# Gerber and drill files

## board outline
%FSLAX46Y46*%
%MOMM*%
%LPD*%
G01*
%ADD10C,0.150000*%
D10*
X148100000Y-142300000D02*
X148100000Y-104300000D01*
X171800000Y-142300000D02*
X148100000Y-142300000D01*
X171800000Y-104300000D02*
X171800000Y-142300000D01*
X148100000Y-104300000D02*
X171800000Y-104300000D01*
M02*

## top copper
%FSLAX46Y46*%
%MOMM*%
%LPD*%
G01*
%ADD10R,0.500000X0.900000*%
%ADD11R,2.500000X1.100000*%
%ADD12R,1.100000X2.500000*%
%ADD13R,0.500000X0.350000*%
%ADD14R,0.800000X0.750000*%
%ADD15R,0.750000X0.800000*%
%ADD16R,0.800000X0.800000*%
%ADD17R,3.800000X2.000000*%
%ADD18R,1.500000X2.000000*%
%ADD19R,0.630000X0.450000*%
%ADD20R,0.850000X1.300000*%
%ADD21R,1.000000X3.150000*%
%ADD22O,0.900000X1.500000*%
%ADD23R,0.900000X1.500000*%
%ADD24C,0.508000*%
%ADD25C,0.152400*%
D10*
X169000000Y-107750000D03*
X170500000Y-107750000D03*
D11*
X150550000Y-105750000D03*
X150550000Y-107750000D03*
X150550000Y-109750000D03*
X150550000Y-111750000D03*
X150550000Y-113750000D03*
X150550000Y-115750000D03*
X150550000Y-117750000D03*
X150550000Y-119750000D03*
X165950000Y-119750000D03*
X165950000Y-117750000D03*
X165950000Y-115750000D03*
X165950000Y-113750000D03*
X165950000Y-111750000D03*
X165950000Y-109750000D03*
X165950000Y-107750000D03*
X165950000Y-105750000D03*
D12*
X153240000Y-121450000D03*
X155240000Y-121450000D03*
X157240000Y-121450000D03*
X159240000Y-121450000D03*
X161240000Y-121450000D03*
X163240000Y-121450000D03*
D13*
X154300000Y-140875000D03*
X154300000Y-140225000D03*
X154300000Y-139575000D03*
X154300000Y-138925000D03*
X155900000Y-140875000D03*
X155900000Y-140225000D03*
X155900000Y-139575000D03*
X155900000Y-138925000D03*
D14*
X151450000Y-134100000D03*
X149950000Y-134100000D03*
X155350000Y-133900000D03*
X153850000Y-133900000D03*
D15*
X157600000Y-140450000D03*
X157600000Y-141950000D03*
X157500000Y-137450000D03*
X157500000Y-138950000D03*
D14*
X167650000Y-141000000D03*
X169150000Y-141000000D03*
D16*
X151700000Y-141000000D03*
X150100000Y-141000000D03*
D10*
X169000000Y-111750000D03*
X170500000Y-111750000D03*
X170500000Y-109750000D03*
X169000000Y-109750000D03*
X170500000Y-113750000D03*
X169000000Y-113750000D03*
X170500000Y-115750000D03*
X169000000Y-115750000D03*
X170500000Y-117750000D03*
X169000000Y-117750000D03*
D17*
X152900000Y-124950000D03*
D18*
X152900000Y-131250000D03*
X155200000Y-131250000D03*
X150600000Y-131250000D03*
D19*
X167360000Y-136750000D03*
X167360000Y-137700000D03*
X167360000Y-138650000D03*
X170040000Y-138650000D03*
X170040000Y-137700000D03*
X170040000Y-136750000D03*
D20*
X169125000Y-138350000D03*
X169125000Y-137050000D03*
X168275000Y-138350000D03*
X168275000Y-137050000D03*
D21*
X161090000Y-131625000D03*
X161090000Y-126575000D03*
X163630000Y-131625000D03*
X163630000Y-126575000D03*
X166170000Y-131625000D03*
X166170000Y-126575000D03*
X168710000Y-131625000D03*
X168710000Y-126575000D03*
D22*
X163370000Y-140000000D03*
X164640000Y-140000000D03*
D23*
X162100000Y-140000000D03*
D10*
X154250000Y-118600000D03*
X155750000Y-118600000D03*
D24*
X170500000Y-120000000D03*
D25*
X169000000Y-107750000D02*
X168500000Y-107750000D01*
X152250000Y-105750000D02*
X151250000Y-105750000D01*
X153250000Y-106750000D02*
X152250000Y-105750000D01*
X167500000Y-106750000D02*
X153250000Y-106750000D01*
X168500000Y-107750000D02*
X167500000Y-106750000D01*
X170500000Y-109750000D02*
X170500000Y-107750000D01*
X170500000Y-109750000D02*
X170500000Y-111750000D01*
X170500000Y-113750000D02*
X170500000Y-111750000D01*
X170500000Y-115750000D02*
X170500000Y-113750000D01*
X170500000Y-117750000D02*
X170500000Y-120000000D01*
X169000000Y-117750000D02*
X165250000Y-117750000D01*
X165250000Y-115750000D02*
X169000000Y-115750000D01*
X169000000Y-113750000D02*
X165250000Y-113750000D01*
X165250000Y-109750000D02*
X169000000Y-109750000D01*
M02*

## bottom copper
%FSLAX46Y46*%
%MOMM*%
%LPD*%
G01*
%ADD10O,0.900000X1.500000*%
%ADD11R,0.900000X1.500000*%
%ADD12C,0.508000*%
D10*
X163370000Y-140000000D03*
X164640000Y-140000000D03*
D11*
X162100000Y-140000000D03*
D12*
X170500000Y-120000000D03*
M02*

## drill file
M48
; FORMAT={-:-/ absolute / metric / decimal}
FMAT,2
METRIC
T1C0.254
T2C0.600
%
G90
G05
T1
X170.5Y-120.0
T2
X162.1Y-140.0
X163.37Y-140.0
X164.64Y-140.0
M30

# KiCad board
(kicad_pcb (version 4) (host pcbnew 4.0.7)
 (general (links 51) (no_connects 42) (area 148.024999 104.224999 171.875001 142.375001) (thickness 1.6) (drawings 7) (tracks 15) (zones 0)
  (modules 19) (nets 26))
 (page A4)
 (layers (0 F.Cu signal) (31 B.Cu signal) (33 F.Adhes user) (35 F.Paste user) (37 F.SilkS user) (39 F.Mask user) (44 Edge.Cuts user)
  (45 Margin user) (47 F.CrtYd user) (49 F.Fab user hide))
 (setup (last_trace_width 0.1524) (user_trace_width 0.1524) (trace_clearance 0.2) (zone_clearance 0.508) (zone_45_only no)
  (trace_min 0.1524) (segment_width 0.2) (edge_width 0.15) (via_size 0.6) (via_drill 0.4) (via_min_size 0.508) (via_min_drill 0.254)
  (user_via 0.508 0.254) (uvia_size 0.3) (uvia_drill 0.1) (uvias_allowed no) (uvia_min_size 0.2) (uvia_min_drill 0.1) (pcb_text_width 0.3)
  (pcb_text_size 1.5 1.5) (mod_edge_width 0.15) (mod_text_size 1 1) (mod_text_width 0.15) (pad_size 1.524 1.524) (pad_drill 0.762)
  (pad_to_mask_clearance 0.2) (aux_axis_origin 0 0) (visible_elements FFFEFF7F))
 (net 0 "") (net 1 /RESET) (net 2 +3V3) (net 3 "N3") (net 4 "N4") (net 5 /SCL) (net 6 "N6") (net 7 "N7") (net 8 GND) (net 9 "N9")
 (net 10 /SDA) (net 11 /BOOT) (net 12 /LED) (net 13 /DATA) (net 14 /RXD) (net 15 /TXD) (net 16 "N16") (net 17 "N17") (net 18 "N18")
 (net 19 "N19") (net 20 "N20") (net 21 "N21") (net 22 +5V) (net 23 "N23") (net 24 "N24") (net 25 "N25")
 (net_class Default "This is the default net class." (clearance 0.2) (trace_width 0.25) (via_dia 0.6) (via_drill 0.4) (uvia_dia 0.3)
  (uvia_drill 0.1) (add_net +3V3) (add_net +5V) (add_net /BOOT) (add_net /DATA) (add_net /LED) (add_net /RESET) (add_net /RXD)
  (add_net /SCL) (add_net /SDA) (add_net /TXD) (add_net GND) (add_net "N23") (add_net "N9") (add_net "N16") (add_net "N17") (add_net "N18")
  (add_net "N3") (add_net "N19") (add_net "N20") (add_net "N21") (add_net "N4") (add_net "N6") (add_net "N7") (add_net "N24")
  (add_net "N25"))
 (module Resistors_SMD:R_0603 (layer F.Cu) (at 169.75 107.75)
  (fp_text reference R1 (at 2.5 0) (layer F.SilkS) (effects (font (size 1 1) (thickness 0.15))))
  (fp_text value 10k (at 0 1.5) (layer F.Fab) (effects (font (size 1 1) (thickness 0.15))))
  (pad 1 smd rect (at -0.75 0) (size 0.5 0.9) (layers F.Cu F.Paste F.Mask) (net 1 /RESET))
  (pad 2 smd rect (at 0.75 0) (size 0.5 0.9) (layers F.Cu F.Paste F.Mask) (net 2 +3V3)))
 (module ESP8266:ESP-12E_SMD (layer F.Cu) (at 151.25 105.75)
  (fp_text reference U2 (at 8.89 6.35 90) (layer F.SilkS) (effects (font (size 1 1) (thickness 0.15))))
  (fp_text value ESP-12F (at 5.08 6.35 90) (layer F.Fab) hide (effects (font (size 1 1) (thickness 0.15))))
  (pad 1 smd rect (at 0 0) (size 2.5 1.1) (drill (offset -0.7 0)) (layers F.Cu F.Paste F.Mask) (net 1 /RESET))
  (pad 2 smd rect (at 0 2) (size 2.5 1.1) (drill (offset -0.7 0)) (layers F.Cu F.Paste F.Mask) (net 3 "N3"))
  (pad 3 smd rect (at 0 4) (size 2.5 1.1) (drill (offset -0.7 0)) (layers F.Cu F.Paste F.Mask) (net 2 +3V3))
  (pad 4 smd rect (at 0 6) (size 2.5 1.1) (drill (offset -0.7 0)) (layers F.Cu F.Paste F.Mask) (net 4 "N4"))
  (pad 5 smd rect (at 0 8) (size 2.5 1.1) (drill (offset -0.7 0)) (layers F.Cu F.Paste F.Mask) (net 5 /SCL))
  (pad 6 smd rect (at 0 10) (size 2.5 1.1) (drill (offset -0.7 0)) (layers F.Cu F.Paste F.Mask) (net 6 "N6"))
  (pad 7 smd rect (at 0 12) (size 2.5 1.1) (drill (offset -0.7 0)) (layers F.Cu F.Paste F.Mask) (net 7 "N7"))
  (pad 8 smd rect (at 0 14) (size 2.5 1.1) (drill (offset -0.7 0)) (layers F.Cu F.Paste F.Mask) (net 2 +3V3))
  (pad 9 smd rect (at 14 14) (size 2.5 1.1) (drill (offset 0.7 0)) (layers F.Cu F.Paste F.Mask) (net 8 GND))
  (pad 10 smd rect (at 14 12) (size 2.5 1.1) (drill (offset 0.7 0)) (layers F.Cu F.Paste F.Mask) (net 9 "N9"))
  (pad 11 smd rect (at 14 10) (size 2.5 1.1) (drill (offset 0.7 0)) (layers F.Cu F.Paste F.Mask) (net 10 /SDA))
  (pad 12 smd rect (at 14 8) (size 2.5 1.1) (drill (offset 0.7 0)) (layers F.Cu F.Paste F.Mask) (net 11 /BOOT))
  (pad 13 smd rect (at 14 6) (size 2.5 1.1) (drill (offset 0.7 0)) (layers F.Cu F.Paste F.Mask) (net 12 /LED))
  (pad 14 smd rect (at 14 4) (size 2.5 1.1) (drill (offset 0.7 0)) (layers F.Cu F.Paste F.Mask) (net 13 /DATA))
  (pad 15 smd rect (at 14 2) (size 2.5 1.1) (drill (offset 0.7 0)) (layers F.Cu F.Paste F.Mask) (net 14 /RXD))
  (pad 16 smd rect (at 14 0) (size 2.5 1.1) (drill (offset 0.7 0)) (layers F.Cu F.Paste F.Mask) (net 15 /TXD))
  (pad 17 smd rect (at 1.99 15 90) (size 2.5 1.1) (drill (offset -0.7 0)) (layers F.Cu F.Paste F.Mask) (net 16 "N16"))
  (pad 18 smd rect (at 3.99 15 90) (size 2.5 1.1) (drill (offset -0.7 0)) (layers F.Cu F.Paste F.Mask) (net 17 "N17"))
  (pad 19 smd rect (at 5.99 15 90) (size 2.5 1.1) (drill (offset -0.7 0)) (layers F.Cu F.Paste F.Mask) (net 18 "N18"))
  (pad 20 smd rect (at 7.99 15 90) (size 2.5 1.1) (drill (offset -0.7 0)) (layers F.Cu F.Paste F.Mask) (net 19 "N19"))
  (pad 21 smd rect (at 9.99 15 90) (size 2.5 1.1) (drill (offset -0.7 0)) (layers F.Cu F.Paste F.Mask) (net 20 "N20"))
  (pad 22 smd rect (at 11.99 15 90) (size 2.5 1.1) (drill (offset -0.7 0)) (layers F.Cu F.Paste F.Mask) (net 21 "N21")))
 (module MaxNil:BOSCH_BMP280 (layer F.Cu) (at 155.1 139.9 90)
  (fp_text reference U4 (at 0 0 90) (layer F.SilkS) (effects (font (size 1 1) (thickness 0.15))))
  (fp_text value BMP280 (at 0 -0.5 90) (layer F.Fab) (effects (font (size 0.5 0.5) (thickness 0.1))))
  (pad 1 smd rect (at -0.975 -0.8 90) (size 0.35 0.5) (layers F.Cu F.Paste F.Mask) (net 8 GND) (solder_mask_margin 0.05))
  (pad 2 smd rect (at -0.325 -0.8 90) (size 0.35 0.5) (layers F.Cu F.Paste F.Mask) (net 2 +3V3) (solder_mask_margin 0.05))
  (pad 3 smd rect (at 0.325 -0.8 90) (size 0.35 0.5) (layers F.Cu F.Paste F.Mask) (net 10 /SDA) (solder_mask_margin 0.05))
  (pad 4 smd rect (at 0.975 -0.8 90) (size 0.35 0.5) (layers F.Cu F.Paste F.Mask) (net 5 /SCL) (solder_mask_margin 0.05))
  (pad 8 smd rect (at -0.975 0.8 90) (size 0.35 0.5) (layers F.Cu F.Paste F.Mask) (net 2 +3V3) (solder_mask_margin 0.05))
  (pad 7 smd rect (at -0.325 0.8 90) (size 0.35 0.5) (layers F.Cu F.Paste F.Mask) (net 8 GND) (solder_mask_margin 0.05))
  (pad 6 smd rect (at 0.325 0.8 90) (size 0.35 0.5) (layers F.Cu F.Paste F.Mask) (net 2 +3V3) (solder_mask_margin 0.05))
  (pad 5 smd rect (at 0.975 0.8 90) (size 0.35 0.5) (layers F.Cu F.Paste F.Mask) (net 8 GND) (solder_mask_margin 0.05)))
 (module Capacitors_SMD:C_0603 (layer F.Cu) (at 150.7 134.1)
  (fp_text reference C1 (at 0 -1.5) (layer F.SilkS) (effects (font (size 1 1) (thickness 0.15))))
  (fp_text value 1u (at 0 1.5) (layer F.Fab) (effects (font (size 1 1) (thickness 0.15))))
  (pad 2 smd rect (at 0.75 0) (size 0.8 0.75) (layers F.Cu F.Paste F.Mask) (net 8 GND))
  (pad 1 smd rect (at -0.75 0) (size 0.8 0.75) (layers F.Cu F.Paste F.Mask) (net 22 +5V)))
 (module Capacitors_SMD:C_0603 (layer F.Cu) (at 154.6 133.9)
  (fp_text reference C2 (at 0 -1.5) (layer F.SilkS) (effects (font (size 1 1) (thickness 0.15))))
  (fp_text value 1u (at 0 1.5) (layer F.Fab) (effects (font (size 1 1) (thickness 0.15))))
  (pad 2 smd rect (at 0.75 0) (size 0.8 0.75) (layers F.Cu F.Paste F.Mask) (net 8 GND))
  (pad 1 smd rect (at -0.75 0) (size 0.8 0.75) (layers F.Cu F.Paste F.Mask) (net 2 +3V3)))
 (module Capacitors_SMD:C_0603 (layer F.Cu) (at 157.6 141.2 90)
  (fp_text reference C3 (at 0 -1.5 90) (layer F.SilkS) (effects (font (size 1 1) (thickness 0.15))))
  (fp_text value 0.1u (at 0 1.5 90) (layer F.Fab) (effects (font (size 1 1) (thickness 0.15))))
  (pad 2 smd rect (at 0.75 0 90) (size 0.8 0.75) (layers F.Cu F.Paste F.Mask) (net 8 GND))
  (pad 1 smd rect (at -0.75 0 90) (size 0.8 0.75) (layers F.Cu F.Paste F.Mask) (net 2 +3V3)))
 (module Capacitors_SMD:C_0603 (layer F.Cu) (at 157.5 138.2 90)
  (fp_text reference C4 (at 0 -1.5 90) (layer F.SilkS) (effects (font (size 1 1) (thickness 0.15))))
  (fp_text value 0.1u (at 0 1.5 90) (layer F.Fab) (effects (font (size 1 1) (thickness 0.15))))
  (pad 2 smd rect (at 0.75 0 90) (size 0.8 0.75) (layers F.Cu F.Paste F.Mask) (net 8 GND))
  (pad 1 smd rect (at -0.75 0 90) (size 0.8 0.75) (layers F.Cu F.Paste F.Mask) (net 2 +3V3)))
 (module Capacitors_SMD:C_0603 (layer F.Cu) (at 168.4 141 180)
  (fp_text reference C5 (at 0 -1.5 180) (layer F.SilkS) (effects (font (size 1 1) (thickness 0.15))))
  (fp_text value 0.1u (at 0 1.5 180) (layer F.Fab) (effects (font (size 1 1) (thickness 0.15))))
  (pad 2 smd rect (at 0.75 0 180) (size 0.8 0.75) (layers F.Cu F.Paste F.Mask) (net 8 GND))
  (pad 1 smd rect (at -0.75 0 180) (size 0.8 0.75) (layers F.Cu F.Paste F.Mask) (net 2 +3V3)))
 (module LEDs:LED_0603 (layer F.Cu) (at 150.9 141)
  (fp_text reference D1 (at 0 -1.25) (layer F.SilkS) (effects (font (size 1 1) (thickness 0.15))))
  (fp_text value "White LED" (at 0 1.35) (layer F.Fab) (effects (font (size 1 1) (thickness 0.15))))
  (pad 2 smd rect (at 0.8 0 180) (size 0.8 0.8) (layers F.Cu F.Paste F.Mask) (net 2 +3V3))
  (pad 1 smd rect (at -0.8 0 180) (size 0.8 0.8) (layers F.Cu F.Paste F.Mask) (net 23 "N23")))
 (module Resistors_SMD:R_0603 (layer F.Cu) (at 169.75 111.75)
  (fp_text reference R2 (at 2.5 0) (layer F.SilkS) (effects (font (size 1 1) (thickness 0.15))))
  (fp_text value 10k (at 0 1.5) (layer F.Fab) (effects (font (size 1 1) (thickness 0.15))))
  (pad 1 smd rect (at -0.75 0) (size 0.5 0.9) (layers F.Cu F.Paste F.Mask) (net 5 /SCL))
  (pad 2 smd rect (at 0.75 0) (size 0.5 0.9) (layers F.Cu F.Paste F.Mask) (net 2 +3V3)))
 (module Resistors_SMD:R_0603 (layer F.Cu) (at 169.75 109.75 180)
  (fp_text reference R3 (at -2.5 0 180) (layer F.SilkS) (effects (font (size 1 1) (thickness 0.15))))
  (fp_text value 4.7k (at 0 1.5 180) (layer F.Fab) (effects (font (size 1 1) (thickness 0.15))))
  (pad 1 smd rect (at -0.75 0 180) (size 0.5 0.9) (layers F.Cu F.Paste F.Mask) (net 2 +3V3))
  (pad 2 smd rect (at 0.75 0 180) (size 0.5 0.9) (layers F.Cu F.Paste F.Mask) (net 13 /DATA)))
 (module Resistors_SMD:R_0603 (layer F.Cu) (at 169.75 113.75 180)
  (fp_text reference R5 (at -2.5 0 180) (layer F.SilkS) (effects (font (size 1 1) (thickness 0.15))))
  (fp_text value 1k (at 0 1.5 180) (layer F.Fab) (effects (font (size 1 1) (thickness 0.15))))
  (pad 1 smd rect (at -0.75 0 180) (size 0.5 0.9) (layers F.Cu F.Paste F.Mask) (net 2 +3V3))
  (pad 2 smd rect (at 0.75 0 180) (size 0.5 0.9) (layers F.Cu F.Paste F.Mask) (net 11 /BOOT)))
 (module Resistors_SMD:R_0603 (layer F.Cu) (at 169.75 115.75 180)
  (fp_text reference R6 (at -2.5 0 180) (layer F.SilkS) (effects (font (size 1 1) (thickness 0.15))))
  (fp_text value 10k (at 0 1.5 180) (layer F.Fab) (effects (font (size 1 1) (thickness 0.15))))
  (pad 1 smd rect (at -0.75 0 180) (size 0.5 0.9) (layers F.Cu F.Paste F.Mask) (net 2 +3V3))
  (pad 2 smd rect (at 0.75 0 180) (size 0.5 0.9) (layers F.Cu F.Paste F.Mask) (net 10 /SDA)))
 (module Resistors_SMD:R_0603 (layer F.Cu) (at 169.75 117.75 180)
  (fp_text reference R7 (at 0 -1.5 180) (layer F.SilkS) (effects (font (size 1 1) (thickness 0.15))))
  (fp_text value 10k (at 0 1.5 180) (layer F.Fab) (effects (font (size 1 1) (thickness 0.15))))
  (pad 1 smd rect (at -0.75 0 180) (size 0.5 0.9) (layers F.Cu F.Paste F.Mask) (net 8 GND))
  (pad 2 smd rect (at 0.75 0 180) (size 0.5 0.9) (layers F.Cu F.Paste F.Mask) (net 9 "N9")))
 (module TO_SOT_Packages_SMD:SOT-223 (layer F.Cu) (at 152.9 128.1 90)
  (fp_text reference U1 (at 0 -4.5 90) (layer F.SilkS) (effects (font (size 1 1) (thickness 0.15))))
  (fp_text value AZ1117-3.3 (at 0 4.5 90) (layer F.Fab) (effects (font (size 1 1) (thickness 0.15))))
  (pad 4 smd rect (at 3.15 0 90) (size 2 3.8) (layers F.Cu F.Paste F.Mask))
  (pad 2 smd rect (at -3.15 0 90) (size 2 1.5) (layers F.Cu F.Paste F.Mask) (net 2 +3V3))
  (pad 3 smd rect (at -3.15 2.3 90) (size 2 1.5) (layers F.Cu F.Paste F.Mask) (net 22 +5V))
  (pad 1 smd rect (at -3.15 -2.3 90) (size 2 1.5) (layers F.Cu F.Paste F.Mask) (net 8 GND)))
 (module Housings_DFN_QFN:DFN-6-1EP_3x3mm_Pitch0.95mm (layer F.Cu) (at 168.7 137.7)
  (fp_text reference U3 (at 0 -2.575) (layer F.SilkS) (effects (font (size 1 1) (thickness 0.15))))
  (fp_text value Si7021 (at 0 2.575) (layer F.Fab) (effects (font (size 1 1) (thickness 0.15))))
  (pad 1 smd rect (at -1.34 -0.95) (size 0.63 0.45) (layers F.Cu F.Paste F.Mask) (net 10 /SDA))
  (pad 2 smd rect (at -1.34 0) (size 0.63 0.45) (layers F.Cu F.Paste F.Mask) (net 8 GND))
  (pad 3 smd rect (at -1.34 0.95) (size 0.63 0.45) (layers F.Cu F.Paste F.Mask) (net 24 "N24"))
  (pad 4 smd rect (at 1.34 0.95) (size 0.63 0.45) (layers F.Cu F.Paste F.Mask) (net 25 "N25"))
  (pad 5 smd rect (at 1.34 0) (size 0.63 0.45) (layers F.Cu F.Paste F.Mask) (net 2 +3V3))
  (pad 6 smd rect (at 1.34 -0.95) (size 0.63 0.45) (layers F.Cu F.Paste F.Mask) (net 5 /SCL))
  (pad 7 smd rect (at 0.425 0.65) (size 0.85 1.3) (layers F.Cu F.Paste F.Mask) (solder_paste_margin_ratio -0.2))
  (pad 7 smd rect (at 0.425 -0.65) (size 0.85 1.3) (layers F.Cu F.Paste F.Mask) (solder_paste_margin_ratio -0.2))
  (pad 7 smd rect (at -0.425 0.65) (size 0.85 1.3) (layers F.Cu F.Paste F.Mask) (solder_paste_margin_ratio -0.2))
  (pad 7 smd rect (at -0.425 -0.65) (size 0.85 1.3) (layers F.Cu F.Paste F.Mask) (solder_paste_margin_ratio -0.2)))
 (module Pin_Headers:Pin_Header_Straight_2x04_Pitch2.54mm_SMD (layer F.Cu) (at 164.9 129.1 90)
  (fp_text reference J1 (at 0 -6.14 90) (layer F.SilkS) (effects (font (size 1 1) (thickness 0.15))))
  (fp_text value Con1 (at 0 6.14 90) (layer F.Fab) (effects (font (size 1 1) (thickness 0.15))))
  (pad 1 smd rect (at -2.525 -3.81 90) (size 3.15 1) (layers F.Cu F.Paste F.Mask) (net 1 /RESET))
  (pad 2 smd rect (at 2.525 -3.81 90) (size 3.15 1) (layers F.Cu F.Paste F.Mask) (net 8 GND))
  (pad 3 smd rect (at -2.525 -1.27 90) (size 3.15 1) (layers F.Cu F.Paste F.Mask) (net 11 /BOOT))
  (pad 4 smd rect (at 2.525 -1.27 90) (size 3.15 1) (layers F.Cu F.Paste F.Mask) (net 8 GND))
  (pad 5 smd rect (at -2.525 1.27 90) (size 3.15 1) (layers F.Cu F.Paste F.Mask) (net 14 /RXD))
  (pad 6 smd rect (at 2.525 1.27 90) (size 3.15 1) (layers F.Cu F.Paste F.Mask) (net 15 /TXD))
  (pad 7 smd rect (at -2.525 3.81 90) (size 3.15 1) (layers F.Cu F.Paste F.Mask) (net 22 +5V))
  (pad 8 smd rect (at 2.525 3.81 90) (size 3.15 1) (layers F.Cu F.Paste F.Mask) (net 8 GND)))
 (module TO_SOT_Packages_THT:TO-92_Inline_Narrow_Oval (layer F.Cu) (at 162.1 140)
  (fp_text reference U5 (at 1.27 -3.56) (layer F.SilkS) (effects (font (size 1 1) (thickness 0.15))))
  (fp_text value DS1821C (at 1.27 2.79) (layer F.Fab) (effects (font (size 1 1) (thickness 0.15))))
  (pad 2 thru_hole oval (at 1.27 0 180) (size 0.9 1.5) (drill 0.6) (layers *.Cu *.Mask) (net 13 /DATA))
  (pad 3 thru_hole oval (at 2.54 0 180) (size 0.9 1.5) (drill 0.6) (layers *.Cu *.Mask) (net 2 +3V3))
  (pad 1 thru_hole rect (at 0 0 180) (size 0.9 1.5) (drill 0.6) (layers *.Cu *.Mask) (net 8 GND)))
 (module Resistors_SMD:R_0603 (layer F.Cu) (at 155 118.6)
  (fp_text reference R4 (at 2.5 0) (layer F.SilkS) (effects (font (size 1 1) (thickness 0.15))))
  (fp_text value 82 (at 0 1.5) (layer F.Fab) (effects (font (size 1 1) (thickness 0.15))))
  (pad 1 smd rect (at -0.75 0) (size 0.5 0.9) (layers F.Cu F.Paste F.Mask) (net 12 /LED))
  (pad 2 smd rect (at 0.75 0) (size 0.5 0.9) (layers F.Cu F.Paste F.Mask) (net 23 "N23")))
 (gr_line (start 148.1 142.3) (end 148.1 104.3) (angle 90) (layer Edge.Cuts) (width 0.15))
 (gr_line (start 171.8 142.3) (end 148.1 142.3) (angle 90) (layer Edge.Cuts) (width 0.15))
 (gr_line (start 171.8 104.3) (end 171.8 142.3) (angle 90) (layer Edge.Cuts) (width 0.15))
 (gr_line (start 148.1 104.3) (end 171.8 104.3) (angle 90) (layer Edge.Cuts) (width 0.15))
 (segment (start 169 107.75) (end 168.5 107.75) (width 0.1524) (layer F.Cu) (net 1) (status 400000))
 (segment (start 152.25 105.75) (end 151.25 105.75) (width 0.1524) (layer F.Cu) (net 1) (status 800000))
 (segment (start 153.25 106.75) (end 152.25 105.75) (width 0.1524) (layer F.Cu) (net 1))
 (segment (start 167.5 106.75) (end 153.25 106.75) (width 0.1524) (layer F.Cu) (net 1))
 (segment (start 168.5 107.75) (end 167.5 106.75) (width 0.1524) (layer F.Cu) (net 1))
 (segment (start 170.5 109.75) (end 170.5 107.75) (width 0.1524) (layer F.Cu) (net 2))
 (segment (start 170.5 109.75) (end 170.5 111.75) (width 0.1524) (layer F.Cu) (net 2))
 (segment (start 170.5 113.75) (end 170.5 111.75) (width 0.1524) (layer F.Cu) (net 2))
 (segment (start 170.5 115.75) (end 170.5 113.75) (width 0.1524) (layer F.Cu) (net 2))
 (segment (start 170.5 117.75) (end 170.5 120) (width 0.1524) (layer F.Cu) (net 8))
 (via (at 170.5 120) (size 0.508) (drill 0.254) (layers F.Cu B.Cu) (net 8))
 (segment (start 169 117.75) (end 165.25 117.75) (width 0.1524) (layer F.Cu) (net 9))
 (segment (start 165.25 115.75) (end 169 115.75) (width 0.1524) (layer F.Cu) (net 10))
 (segment (start 169 113.75) (end 165.25 113.75) (width 0.1524) (layer F.Cu) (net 11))
 (segment (start 165.25 109.75) (end 169 109.75) (width 0.1524) (layer F.Cu) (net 13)))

